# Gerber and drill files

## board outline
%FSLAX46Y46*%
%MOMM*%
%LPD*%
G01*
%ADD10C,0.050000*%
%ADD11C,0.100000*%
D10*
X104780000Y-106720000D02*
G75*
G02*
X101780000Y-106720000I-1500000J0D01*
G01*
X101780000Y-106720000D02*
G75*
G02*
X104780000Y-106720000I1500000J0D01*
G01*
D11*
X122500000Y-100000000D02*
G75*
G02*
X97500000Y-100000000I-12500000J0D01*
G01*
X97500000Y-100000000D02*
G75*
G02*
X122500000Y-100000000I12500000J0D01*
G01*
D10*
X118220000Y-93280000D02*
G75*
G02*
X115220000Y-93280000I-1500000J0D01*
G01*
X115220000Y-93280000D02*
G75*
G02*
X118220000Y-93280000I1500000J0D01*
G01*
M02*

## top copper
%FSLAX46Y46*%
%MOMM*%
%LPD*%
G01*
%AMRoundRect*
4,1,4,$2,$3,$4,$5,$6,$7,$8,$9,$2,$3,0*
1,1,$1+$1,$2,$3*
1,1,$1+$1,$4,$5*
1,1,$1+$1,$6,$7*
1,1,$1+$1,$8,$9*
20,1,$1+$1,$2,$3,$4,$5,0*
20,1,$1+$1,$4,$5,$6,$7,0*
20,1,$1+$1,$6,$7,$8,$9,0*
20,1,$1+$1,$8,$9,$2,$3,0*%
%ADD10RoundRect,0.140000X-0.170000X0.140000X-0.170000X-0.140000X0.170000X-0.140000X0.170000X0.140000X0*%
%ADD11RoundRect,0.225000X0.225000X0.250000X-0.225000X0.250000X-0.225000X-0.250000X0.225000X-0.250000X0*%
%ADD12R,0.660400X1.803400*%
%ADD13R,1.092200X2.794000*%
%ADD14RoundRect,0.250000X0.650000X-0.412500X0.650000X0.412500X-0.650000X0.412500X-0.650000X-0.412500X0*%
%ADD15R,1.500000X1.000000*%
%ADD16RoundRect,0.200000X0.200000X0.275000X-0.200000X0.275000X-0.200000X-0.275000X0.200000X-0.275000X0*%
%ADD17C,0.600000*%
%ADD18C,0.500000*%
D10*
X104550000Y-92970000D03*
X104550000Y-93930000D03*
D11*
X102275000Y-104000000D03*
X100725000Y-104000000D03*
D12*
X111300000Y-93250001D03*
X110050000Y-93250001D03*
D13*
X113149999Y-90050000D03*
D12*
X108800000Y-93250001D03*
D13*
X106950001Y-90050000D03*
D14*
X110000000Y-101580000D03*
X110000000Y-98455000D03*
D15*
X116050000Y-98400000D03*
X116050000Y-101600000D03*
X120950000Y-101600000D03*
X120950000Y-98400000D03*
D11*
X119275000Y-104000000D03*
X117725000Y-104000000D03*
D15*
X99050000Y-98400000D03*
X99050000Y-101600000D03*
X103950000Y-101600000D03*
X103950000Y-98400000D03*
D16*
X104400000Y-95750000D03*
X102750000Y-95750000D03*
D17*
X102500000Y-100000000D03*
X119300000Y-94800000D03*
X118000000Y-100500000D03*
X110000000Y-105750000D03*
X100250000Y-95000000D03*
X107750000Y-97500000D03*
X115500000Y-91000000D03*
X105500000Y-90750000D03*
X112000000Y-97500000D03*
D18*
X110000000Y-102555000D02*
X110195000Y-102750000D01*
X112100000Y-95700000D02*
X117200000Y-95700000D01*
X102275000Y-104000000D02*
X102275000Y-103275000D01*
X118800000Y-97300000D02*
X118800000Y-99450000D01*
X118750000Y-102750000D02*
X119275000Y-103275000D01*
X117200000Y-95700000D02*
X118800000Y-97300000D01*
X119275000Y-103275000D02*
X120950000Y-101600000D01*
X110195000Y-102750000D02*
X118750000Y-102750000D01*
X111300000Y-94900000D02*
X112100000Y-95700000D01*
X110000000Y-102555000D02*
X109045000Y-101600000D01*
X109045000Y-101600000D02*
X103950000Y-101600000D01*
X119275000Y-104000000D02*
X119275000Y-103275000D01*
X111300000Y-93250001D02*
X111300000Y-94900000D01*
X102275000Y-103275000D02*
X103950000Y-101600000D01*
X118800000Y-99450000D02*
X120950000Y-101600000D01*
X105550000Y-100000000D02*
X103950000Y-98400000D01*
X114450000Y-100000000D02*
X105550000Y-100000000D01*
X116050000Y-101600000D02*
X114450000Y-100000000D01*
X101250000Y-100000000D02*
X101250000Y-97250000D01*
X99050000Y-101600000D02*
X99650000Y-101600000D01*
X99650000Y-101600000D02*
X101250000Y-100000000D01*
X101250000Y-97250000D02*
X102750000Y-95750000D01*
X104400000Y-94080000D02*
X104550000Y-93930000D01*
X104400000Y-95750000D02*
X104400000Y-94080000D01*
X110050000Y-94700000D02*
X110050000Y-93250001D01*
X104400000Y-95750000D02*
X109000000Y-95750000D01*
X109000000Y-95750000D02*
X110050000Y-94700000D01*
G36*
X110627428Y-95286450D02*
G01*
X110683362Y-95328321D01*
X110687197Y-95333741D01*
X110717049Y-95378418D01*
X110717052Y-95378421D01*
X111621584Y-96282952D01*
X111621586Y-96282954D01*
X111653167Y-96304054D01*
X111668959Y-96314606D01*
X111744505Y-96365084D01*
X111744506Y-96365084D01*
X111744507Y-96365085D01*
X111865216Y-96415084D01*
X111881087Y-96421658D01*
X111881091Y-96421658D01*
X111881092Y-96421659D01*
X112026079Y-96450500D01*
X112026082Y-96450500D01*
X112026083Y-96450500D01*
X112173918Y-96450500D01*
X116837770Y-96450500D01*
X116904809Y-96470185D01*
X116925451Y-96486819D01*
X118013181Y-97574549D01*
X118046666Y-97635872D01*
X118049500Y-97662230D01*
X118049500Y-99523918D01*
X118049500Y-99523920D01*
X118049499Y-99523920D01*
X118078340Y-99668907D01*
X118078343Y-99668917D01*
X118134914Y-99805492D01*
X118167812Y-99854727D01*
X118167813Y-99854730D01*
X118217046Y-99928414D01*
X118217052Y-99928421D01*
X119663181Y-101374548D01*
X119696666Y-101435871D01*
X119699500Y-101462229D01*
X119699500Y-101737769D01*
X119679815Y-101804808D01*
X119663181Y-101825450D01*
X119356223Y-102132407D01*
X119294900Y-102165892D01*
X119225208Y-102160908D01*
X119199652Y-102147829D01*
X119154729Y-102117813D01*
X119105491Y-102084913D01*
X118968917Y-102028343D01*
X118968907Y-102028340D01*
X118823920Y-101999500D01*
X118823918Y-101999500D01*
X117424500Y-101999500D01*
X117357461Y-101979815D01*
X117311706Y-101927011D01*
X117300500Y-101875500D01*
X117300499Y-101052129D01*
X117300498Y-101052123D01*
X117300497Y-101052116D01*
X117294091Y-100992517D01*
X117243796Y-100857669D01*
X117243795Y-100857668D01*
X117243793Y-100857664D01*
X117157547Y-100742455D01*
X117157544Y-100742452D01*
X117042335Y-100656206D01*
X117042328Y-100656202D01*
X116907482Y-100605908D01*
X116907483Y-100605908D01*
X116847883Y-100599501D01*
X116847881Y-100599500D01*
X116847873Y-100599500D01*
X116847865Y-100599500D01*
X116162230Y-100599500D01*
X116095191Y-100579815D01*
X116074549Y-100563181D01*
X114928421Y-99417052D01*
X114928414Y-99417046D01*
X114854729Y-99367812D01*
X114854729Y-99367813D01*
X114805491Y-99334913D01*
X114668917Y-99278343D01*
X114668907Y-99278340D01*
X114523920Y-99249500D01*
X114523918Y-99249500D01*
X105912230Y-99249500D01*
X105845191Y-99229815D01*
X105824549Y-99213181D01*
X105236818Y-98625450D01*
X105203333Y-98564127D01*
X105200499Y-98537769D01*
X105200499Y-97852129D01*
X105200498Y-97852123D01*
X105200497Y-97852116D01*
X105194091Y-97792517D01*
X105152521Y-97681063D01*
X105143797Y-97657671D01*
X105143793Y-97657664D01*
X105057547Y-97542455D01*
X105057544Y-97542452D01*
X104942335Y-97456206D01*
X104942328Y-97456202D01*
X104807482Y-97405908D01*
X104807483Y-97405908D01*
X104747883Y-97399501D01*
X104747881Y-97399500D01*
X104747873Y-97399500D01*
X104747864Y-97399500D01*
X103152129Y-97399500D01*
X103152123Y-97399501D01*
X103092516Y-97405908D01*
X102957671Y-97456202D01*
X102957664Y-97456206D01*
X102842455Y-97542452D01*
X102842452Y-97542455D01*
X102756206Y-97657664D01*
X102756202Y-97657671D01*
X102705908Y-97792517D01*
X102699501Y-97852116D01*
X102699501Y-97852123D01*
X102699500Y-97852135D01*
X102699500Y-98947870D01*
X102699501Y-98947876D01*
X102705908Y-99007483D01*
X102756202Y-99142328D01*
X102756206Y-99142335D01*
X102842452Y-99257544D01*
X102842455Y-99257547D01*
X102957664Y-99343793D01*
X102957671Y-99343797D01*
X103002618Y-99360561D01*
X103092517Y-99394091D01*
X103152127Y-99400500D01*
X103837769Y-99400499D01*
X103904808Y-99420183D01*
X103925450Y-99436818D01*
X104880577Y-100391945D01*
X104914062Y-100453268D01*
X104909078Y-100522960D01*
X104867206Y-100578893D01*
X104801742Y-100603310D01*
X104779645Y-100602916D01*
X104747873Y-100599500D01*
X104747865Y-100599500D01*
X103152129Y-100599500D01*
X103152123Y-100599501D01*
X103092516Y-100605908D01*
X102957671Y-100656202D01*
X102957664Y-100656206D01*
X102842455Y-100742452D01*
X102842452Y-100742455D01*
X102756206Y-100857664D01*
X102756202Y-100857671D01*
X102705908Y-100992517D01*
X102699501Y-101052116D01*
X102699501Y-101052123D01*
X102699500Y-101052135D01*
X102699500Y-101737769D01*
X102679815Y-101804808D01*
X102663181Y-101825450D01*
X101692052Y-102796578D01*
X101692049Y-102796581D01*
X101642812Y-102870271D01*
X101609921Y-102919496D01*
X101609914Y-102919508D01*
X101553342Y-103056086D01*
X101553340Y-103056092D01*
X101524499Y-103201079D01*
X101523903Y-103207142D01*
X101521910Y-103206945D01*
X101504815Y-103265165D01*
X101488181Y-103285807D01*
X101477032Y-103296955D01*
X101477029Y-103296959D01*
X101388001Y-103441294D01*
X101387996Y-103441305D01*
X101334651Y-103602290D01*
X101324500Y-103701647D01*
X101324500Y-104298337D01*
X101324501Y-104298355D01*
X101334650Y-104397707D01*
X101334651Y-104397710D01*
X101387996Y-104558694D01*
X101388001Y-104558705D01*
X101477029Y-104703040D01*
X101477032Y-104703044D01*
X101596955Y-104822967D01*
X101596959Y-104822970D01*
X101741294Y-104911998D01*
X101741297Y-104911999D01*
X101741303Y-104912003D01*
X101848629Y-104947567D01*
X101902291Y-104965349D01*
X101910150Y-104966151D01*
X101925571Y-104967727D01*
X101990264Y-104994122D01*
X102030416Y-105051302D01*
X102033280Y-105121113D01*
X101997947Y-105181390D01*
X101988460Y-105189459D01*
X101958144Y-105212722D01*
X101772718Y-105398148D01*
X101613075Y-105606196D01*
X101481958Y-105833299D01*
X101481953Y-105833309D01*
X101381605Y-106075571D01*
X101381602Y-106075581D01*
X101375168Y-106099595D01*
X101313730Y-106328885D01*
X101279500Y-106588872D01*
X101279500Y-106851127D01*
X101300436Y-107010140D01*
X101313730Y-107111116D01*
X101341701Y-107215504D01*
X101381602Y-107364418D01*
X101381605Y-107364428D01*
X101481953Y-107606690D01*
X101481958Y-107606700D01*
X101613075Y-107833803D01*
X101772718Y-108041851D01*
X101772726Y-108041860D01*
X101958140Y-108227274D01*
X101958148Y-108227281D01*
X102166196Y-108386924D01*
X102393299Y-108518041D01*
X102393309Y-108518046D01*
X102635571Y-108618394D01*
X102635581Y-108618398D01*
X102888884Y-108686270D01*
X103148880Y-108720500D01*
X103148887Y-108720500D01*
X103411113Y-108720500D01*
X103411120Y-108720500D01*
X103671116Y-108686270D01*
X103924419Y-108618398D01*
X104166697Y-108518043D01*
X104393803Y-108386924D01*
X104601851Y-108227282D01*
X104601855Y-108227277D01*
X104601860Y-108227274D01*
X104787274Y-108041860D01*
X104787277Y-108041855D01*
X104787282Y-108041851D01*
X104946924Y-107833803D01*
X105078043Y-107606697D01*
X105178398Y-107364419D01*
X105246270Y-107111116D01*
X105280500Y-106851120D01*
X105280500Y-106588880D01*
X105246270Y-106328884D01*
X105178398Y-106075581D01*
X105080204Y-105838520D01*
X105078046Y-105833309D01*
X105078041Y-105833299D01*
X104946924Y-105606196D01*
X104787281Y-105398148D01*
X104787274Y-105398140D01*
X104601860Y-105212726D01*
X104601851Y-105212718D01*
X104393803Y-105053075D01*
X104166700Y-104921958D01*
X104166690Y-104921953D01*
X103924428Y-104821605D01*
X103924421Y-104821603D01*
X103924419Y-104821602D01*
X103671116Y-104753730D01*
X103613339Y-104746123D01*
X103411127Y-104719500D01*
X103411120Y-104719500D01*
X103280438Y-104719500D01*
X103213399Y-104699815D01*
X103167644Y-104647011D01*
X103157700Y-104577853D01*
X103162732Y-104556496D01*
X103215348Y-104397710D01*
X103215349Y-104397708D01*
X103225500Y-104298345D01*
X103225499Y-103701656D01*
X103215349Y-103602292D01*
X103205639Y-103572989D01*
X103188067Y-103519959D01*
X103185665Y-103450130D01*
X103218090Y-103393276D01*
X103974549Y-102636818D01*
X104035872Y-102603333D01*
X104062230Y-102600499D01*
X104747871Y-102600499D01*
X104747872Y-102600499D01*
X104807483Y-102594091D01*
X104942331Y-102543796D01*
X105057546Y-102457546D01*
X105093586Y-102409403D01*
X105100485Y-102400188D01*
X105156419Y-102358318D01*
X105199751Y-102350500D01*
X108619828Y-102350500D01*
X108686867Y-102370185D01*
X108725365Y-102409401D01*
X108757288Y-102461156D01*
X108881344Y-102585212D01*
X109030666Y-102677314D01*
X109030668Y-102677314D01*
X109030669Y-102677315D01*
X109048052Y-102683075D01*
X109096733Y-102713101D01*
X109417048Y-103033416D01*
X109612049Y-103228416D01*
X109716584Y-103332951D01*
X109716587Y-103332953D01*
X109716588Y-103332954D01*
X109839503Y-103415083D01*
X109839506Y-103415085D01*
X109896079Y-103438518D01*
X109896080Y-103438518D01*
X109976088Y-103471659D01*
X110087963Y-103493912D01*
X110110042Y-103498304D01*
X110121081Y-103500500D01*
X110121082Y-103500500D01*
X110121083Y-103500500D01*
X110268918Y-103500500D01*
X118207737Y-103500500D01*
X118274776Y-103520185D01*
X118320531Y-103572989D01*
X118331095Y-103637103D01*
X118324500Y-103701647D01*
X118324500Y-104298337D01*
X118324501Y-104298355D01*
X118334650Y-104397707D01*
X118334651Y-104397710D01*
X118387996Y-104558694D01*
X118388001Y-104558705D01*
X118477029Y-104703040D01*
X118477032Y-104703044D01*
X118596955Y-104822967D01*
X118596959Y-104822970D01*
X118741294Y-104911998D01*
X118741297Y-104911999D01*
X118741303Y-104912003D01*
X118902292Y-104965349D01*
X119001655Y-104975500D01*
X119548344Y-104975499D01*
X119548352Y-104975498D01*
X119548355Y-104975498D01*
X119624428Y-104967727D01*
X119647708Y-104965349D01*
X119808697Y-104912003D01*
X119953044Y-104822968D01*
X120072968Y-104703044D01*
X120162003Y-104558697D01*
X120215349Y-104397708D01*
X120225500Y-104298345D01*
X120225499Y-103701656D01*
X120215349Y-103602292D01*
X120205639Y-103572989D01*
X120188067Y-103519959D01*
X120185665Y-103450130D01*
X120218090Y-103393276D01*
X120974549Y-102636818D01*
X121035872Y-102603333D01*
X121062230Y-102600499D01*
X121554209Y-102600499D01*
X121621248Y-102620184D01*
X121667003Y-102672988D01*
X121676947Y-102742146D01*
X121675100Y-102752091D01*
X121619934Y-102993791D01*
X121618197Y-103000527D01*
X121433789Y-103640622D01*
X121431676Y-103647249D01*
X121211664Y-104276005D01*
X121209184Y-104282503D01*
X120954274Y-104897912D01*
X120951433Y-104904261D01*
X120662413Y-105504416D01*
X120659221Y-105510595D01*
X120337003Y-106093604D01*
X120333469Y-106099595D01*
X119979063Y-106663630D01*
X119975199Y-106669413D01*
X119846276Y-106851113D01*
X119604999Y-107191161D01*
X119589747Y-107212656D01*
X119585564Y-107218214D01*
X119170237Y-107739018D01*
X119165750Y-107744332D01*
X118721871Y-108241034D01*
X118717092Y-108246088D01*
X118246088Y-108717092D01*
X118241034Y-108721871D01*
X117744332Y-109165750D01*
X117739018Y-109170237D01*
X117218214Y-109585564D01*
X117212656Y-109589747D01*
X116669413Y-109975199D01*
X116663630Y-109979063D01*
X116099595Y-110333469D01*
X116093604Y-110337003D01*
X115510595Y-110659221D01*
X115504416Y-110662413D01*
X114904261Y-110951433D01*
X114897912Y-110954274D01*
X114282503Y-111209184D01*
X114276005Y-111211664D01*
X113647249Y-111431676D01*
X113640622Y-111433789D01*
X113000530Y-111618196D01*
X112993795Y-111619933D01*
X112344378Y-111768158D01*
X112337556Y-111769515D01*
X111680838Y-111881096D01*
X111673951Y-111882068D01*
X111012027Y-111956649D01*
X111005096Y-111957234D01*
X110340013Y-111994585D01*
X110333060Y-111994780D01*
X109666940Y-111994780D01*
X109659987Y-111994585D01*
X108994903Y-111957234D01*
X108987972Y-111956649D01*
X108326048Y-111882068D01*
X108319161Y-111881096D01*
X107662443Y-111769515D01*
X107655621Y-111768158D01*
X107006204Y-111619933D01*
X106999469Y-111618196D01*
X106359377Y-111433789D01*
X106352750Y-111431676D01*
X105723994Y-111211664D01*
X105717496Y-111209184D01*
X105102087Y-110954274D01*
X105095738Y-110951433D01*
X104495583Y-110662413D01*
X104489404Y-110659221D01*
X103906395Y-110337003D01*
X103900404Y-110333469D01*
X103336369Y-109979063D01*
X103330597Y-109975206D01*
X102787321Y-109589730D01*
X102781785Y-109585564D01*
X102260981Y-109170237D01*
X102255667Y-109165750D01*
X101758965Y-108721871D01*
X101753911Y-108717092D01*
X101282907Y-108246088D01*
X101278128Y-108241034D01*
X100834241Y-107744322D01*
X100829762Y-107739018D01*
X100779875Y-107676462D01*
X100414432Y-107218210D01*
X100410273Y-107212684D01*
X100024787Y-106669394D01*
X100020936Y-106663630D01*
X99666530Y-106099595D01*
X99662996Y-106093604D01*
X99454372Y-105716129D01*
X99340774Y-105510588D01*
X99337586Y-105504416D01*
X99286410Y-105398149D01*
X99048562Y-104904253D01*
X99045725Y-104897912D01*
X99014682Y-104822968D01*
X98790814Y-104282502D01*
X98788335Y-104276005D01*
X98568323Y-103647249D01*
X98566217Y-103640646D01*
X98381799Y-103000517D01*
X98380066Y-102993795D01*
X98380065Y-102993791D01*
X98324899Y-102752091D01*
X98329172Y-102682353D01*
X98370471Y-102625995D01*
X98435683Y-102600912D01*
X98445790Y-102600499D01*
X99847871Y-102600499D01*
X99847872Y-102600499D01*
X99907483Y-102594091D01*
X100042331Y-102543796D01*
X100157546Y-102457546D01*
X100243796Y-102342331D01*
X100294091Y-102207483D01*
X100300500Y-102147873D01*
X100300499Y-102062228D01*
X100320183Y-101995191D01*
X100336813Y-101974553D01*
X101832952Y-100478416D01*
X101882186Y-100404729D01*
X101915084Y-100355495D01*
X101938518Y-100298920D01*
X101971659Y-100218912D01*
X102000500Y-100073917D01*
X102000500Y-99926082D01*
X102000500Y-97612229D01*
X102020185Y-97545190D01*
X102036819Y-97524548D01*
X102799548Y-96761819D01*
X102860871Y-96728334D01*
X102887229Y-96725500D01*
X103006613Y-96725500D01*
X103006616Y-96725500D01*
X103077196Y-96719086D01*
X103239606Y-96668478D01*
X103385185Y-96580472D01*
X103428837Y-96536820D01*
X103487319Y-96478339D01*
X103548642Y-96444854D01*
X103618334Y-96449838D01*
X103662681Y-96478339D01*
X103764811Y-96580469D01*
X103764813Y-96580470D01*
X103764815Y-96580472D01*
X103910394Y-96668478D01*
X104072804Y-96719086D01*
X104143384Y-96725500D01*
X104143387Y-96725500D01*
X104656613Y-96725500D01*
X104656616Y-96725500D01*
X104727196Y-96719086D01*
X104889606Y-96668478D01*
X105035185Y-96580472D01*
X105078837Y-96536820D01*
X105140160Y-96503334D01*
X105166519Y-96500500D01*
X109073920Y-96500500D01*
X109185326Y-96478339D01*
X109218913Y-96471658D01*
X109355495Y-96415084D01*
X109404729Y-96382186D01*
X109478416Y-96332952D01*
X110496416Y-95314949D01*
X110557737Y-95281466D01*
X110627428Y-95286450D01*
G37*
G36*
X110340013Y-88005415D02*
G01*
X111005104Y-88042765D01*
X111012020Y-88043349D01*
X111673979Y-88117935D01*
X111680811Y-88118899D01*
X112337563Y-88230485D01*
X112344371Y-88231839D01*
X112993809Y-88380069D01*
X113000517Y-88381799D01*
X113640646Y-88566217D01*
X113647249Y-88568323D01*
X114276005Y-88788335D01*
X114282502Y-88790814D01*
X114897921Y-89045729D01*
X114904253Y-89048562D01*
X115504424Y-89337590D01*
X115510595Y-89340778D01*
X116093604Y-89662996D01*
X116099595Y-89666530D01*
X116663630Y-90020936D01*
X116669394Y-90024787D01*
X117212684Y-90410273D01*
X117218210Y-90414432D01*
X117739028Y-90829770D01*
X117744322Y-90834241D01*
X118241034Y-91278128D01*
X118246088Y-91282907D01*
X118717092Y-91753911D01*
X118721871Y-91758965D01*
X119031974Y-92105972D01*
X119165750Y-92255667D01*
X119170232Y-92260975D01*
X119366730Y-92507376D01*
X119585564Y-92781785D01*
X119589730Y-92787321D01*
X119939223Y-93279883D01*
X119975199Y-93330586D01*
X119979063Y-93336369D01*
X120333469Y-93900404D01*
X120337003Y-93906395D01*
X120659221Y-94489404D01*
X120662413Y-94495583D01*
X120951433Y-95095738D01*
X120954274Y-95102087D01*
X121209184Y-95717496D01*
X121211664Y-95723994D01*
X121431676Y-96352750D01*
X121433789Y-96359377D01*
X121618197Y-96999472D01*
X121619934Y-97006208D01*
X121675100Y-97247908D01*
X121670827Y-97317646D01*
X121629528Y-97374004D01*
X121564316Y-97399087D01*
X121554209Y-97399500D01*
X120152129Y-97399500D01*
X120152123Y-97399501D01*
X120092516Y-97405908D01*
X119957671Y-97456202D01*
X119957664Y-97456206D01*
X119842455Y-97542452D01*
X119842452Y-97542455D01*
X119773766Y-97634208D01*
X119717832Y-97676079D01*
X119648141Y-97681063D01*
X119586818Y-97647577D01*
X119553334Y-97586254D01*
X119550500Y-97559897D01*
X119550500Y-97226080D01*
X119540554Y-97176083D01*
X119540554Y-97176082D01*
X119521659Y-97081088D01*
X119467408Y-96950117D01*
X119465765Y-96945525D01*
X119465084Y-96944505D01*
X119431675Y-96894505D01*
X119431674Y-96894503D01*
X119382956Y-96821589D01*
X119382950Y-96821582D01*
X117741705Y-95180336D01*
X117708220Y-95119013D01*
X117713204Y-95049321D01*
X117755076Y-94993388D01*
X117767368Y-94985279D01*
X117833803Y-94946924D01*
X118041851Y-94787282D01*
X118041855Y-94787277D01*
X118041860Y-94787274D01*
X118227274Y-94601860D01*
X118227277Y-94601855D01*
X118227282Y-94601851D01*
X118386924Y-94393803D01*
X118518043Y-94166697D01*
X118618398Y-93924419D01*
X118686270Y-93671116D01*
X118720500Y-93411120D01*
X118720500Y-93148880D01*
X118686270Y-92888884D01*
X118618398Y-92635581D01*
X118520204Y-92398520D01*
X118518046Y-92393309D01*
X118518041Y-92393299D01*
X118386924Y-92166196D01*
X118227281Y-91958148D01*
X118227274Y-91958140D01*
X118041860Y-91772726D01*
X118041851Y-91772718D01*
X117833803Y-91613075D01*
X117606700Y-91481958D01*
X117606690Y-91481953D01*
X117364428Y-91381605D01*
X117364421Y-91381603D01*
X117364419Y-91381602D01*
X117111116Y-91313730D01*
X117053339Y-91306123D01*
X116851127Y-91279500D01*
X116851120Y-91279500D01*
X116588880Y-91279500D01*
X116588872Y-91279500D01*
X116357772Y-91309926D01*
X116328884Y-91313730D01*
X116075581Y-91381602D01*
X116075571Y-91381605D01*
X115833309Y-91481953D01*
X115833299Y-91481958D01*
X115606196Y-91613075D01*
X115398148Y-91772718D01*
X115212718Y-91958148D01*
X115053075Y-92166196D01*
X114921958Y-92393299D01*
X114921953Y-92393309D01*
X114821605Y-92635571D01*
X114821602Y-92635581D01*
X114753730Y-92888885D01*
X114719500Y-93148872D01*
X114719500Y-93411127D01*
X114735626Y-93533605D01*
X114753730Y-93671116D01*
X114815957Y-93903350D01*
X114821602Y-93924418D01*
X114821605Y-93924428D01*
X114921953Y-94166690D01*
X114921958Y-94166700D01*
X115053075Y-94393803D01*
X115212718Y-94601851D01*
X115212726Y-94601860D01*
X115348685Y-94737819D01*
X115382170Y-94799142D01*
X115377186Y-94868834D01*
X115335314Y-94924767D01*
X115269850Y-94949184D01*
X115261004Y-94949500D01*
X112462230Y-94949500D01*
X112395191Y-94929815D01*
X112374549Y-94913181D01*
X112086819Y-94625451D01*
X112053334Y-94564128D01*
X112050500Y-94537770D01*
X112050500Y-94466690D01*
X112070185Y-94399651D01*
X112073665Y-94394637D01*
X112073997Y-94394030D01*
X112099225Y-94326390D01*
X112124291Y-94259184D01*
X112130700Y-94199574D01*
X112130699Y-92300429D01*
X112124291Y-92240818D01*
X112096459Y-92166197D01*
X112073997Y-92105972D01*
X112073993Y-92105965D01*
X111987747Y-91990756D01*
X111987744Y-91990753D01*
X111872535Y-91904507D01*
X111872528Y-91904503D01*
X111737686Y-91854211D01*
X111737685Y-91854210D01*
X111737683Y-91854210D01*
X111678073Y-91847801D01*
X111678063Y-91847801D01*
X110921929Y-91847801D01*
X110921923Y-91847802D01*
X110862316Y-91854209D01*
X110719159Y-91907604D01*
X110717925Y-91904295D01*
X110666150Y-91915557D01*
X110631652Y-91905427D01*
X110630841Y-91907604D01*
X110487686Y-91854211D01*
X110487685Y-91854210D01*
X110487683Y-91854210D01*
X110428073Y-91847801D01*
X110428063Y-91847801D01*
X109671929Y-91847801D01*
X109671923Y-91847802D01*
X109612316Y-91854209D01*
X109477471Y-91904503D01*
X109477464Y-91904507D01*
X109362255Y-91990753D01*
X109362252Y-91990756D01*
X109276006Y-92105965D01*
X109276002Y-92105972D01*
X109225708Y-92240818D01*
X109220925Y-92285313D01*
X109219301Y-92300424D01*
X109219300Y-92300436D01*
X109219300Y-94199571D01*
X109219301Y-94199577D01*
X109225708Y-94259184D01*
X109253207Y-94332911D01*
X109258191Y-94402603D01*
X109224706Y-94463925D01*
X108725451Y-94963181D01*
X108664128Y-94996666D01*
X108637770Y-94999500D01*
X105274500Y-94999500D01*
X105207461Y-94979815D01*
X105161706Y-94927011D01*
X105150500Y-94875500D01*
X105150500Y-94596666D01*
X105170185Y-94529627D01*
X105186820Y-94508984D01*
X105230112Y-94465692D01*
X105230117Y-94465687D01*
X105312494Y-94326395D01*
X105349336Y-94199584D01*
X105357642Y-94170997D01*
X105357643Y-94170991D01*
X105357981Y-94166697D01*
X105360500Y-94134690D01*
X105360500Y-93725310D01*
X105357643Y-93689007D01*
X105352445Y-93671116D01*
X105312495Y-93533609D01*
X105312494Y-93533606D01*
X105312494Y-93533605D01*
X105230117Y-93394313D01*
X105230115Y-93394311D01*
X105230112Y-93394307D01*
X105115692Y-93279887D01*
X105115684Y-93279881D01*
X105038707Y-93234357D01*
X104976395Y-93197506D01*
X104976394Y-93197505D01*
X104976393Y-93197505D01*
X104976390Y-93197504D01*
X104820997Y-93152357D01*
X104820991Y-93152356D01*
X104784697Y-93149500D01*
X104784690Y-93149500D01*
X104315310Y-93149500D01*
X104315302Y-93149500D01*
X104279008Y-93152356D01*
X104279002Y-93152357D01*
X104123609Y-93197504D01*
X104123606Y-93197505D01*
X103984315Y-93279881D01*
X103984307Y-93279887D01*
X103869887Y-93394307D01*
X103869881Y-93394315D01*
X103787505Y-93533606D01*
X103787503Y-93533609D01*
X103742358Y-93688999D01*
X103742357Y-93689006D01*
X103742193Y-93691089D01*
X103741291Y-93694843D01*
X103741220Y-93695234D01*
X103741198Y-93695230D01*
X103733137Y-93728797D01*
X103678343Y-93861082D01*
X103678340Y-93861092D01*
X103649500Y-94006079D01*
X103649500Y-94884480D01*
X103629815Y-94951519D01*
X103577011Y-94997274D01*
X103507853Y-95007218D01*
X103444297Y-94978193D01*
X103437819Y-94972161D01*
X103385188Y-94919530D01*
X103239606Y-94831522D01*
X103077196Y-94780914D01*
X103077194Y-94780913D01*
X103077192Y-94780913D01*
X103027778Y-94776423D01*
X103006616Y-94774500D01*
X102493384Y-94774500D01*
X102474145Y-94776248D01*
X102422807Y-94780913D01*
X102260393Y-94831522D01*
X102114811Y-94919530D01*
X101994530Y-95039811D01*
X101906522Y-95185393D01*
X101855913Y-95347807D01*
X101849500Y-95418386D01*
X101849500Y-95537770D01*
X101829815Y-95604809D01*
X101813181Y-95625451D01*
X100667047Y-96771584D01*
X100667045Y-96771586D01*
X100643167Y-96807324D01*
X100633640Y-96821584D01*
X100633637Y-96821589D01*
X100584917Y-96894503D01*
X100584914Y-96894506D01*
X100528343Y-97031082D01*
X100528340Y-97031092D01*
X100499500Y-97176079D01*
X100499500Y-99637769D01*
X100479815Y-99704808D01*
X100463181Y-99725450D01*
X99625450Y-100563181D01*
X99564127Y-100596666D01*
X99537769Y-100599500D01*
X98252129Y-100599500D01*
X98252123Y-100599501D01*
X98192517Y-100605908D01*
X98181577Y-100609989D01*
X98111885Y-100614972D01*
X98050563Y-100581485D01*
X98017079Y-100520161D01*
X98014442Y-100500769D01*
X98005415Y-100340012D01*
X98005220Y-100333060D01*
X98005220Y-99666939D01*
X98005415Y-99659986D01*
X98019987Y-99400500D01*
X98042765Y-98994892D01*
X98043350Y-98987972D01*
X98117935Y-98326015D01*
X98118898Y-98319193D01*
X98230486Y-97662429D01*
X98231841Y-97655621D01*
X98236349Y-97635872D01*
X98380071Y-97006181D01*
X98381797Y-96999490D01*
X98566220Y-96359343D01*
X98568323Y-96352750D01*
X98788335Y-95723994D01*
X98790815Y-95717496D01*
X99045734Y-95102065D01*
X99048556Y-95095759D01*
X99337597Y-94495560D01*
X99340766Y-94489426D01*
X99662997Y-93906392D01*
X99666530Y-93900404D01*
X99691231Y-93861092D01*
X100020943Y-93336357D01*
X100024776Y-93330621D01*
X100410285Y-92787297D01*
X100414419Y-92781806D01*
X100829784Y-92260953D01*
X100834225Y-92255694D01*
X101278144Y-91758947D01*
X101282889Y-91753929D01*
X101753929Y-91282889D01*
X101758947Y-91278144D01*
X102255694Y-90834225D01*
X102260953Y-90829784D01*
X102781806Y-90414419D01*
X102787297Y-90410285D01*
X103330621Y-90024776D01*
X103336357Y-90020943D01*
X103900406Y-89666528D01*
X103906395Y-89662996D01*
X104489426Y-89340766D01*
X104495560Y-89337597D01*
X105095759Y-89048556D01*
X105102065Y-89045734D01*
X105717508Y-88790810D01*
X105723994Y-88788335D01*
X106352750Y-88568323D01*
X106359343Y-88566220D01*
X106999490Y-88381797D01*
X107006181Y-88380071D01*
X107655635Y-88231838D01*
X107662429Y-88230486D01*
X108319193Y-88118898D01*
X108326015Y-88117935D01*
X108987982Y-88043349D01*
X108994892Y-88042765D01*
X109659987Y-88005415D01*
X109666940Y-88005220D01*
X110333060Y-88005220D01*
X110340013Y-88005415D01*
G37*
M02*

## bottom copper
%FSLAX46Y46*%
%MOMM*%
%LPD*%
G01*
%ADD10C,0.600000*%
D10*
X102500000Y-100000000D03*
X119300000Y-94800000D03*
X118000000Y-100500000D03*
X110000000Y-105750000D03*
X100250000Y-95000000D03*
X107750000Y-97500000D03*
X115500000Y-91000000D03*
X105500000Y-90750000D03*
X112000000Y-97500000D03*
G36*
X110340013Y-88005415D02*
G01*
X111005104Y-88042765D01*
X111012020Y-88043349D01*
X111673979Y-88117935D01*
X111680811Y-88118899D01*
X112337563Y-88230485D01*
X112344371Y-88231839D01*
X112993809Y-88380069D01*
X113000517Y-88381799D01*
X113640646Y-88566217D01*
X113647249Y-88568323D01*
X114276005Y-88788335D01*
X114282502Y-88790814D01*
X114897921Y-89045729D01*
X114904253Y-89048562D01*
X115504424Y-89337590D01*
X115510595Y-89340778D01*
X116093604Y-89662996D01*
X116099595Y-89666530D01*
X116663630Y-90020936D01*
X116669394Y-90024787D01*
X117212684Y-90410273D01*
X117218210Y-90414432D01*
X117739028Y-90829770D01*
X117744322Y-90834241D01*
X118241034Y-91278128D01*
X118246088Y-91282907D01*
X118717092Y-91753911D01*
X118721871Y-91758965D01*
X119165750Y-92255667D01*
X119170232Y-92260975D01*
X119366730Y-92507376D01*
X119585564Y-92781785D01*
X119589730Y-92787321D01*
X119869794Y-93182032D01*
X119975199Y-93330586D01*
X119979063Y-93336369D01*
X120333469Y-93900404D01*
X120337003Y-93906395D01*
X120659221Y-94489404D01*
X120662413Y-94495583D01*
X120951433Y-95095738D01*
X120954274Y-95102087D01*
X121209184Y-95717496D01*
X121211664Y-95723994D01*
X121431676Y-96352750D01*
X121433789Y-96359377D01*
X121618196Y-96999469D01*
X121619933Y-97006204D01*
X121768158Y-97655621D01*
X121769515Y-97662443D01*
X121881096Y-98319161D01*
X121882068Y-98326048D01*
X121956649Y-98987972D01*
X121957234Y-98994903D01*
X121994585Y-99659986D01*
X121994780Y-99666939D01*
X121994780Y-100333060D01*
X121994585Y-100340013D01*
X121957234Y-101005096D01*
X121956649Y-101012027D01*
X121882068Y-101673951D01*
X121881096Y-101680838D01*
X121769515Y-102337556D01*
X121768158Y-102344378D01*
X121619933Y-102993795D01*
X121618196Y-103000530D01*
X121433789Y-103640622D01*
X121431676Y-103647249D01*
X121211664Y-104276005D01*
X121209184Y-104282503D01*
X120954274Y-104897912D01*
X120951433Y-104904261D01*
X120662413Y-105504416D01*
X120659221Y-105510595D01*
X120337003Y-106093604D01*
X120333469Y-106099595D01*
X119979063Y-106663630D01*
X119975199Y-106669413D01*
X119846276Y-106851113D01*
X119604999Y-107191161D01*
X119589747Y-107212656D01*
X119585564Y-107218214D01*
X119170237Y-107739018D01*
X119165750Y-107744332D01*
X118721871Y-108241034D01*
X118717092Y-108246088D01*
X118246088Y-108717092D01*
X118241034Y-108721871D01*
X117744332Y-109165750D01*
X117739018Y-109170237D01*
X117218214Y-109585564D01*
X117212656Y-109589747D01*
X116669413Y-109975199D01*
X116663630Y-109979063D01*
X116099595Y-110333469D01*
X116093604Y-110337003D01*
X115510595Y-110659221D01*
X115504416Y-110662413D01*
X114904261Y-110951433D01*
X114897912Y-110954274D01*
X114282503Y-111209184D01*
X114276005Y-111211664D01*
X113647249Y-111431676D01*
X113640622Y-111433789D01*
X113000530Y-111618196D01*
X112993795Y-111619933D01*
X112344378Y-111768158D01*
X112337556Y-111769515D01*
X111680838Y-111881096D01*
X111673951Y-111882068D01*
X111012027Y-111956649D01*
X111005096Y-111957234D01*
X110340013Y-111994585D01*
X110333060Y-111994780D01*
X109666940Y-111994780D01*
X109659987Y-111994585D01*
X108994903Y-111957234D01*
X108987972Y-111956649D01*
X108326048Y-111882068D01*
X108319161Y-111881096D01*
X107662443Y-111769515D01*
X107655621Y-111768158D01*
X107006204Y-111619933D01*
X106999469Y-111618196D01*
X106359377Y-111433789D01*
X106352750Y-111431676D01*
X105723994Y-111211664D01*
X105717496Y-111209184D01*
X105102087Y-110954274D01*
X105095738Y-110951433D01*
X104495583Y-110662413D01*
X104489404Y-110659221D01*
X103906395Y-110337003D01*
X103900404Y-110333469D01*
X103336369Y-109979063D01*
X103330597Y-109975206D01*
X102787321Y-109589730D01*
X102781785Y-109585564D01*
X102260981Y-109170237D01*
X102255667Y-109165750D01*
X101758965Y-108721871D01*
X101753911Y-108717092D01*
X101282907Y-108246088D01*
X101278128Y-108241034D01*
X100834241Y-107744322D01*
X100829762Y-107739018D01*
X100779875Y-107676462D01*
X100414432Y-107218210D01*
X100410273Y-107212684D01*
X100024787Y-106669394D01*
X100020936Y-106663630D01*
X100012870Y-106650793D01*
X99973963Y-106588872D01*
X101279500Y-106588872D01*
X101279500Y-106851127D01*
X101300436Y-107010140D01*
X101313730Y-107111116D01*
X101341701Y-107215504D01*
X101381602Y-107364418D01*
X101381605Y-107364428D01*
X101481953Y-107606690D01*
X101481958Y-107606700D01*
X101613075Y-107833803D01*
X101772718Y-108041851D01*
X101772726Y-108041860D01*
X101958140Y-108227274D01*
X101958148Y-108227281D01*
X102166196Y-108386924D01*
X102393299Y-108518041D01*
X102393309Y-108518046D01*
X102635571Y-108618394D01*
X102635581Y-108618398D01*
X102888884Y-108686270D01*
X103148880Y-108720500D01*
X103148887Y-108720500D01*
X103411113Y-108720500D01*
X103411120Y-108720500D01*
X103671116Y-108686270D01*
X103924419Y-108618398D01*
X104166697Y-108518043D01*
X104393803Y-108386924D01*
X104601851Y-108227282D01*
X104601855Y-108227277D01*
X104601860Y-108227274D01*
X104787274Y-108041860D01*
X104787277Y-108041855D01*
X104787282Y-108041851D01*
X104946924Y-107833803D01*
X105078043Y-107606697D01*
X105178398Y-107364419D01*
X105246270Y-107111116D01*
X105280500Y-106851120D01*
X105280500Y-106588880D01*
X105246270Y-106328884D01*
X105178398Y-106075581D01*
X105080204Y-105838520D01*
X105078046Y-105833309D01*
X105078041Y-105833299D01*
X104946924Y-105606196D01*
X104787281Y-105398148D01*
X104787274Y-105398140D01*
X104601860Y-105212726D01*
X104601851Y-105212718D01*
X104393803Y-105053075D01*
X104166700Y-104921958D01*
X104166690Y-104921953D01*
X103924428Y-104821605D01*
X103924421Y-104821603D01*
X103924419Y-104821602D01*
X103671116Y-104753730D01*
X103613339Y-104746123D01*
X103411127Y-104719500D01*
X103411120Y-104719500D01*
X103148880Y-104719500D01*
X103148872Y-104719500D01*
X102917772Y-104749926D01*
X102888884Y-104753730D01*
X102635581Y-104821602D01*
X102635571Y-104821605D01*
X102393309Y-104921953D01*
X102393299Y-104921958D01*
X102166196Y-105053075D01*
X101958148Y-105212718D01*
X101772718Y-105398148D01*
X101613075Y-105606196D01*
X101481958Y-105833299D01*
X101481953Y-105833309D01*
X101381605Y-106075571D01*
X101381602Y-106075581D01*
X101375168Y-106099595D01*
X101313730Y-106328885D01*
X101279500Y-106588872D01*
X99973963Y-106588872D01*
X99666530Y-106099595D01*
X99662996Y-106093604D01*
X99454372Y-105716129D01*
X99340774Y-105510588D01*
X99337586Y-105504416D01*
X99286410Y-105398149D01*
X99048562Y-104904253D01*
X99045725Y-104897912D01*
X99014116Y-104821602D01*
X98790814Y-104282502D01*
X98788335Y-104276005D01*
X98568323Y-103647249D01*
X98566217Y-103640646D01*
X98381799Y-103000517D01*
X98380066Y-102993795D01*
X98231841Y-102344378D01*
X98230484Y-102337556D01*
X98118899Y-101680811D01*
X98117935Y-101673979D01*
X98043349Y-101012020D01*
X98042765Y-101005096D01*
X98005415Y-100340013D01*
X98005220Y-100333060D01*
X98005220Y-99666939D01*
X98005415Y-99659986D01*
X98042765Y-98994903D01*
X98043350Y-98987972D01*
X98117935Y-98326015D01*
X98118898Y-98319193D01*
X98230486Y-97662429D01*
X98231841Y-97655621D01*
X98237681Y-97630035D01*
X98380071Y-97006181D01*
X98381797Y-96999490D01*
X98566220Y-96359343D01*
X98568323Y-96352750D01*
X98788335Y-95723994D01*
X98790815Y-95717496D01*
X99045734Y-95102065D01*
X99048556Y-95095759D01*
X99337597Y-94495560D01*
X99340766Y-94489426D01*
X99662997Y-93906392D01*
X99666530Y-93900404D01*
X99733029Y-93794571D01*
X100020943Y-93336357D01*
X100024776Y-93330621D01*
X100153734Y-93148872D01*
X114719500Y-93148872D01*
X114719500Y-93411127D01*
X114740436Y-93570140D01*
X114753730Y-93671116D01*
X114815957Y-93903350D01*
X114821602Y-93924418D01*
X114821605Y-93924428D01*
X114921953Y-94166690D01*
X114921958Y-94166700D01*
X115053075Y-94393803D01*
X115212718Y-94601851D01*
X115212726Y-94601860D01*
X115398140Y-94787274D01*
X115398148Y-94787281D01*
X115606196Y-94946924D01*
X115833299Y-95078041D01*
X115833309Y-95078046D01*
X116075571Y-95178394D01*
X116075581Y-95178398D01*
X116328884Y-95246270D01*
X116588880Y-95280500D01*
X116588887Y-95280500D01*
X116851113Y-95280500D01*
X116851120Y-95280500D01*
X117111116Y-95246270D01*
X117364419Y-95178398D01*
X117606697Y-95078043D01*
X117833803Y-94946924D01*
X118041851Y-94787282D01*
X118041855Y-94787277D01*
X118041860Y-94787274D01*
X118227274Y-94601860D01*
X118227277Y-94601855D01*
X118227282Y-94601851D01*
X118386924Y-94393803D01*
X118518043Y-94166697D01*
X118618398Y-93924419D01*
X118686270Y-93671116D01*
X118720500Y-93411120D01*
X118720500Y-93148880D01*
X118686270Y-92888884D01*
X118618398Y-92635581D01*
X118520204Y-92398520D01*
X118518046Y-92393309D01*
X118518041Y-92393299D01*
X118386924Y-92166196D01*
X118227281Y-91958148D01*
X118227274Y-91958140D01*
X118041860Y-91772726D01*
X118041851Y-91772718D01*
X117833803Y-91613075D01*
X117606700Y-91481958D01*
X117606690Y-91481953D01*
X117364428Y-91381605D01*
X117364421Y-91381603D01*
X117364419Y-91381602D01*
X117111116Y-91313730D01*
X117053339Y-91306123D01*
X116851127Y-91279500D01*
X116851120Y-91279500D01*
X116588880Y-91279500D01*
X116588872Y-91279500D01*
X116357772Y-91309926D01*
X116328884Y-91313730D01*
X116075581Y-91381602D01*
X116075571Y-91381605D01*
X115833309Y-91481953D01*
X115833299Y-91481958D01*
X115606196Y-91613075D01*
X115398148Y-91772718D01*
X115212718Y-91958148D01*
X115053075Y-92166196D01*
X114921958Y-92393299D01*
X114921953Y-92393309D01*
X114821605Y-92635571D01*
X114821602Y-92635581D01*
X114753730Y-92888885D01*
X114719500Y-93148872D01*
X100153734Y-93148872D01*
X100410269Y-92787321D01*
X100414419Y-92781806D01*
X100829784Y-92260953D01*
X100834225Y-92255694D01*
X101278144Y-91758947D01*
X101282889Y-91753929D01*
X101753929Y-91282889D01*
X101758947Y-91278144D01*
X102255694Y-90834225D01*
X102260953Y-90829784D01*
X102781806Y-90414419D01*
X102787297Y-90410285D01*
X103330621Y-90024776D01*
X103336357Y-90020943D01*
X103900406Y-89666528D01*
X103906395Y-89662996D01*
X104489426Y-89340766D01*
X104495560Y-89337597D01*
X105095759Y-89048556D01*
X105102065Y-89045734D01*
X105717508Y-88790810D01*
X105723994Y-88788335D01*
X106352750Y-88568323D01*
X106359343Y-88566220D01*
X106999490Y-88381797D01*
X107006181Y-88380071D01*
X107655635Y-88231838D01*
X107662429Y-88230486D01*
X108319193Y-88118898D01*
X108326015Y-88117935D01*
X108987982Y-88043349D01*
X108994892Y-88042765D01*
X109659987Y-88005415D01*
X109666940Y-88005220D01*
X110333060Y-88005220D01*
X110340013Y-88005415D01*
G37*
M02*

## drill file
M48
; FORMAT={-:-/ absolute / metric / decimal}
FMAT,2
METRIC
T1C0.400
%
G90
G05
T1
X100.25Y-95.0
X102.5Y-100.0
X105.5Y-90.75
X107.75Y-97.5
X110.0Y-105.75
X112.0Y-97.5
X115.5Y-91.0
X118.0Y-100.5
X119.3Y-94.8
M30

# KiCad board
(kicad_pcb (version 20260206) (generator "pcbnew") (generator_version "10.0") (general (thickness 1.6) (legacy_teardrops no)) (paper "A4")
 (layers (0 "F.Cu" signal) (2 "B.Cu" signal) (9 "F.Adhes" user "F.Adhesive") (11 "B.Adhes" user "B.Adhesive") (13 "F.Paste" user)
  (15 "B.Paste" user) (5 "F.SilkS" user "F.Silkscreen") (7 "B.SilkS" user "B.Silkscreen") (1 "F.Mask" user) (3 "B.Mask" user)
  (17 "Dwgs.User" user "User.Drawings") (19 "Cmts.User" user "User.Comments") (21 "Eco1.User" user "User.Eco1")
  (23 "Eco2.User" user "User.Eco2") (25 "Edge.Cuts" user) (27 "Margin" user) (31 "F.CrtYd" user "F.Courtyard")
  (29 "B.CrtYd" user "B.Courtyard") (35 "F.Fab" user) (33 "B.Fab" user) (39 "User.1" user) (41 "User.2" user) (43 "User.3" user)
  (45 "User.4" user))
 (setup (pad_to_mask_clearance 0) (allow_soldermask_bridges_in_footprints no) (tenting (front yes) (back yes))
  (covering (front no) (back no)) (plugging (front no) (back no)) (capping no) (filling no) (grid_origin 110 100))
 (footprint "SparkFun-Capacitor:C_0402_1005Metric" (layer "F.Cu") (at 104.55 93.45 -90)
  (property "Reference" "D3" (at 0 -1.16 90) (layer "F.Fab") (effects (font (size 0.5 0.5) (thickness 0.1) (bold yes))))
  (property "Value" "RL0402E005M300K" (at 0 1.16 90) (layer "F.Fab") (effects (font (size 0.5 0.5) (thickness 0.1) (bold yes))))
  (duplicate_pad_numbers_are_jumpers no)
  (pad "1" smd roundrect (at -0.48 0 270) (size 0.56 0.62) (layers "F.Cu" "F.Mask" "F.Paste") (roundrect_rratio 0.25) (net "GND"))
  (pad "2" smd roundrect (at 0.48 0 270) (size 0.56 0.62) (layers "F.Cu" "F.Mask" "F.Paste") (roundrect_rratio 0.25) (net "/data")))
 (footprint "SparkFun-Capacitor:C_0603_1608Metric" (layer "F.Cu") (at 101.5 104 180)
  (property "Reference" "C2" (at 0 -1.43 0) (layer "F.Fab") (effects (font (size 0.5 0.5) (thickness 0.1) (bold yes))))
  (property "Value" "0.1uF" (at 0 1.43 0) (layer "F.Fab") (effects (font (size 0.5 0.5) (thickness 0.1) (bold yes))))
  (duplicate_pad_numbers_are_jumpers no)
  (pad "1" smd roundrect (at -0.775 0 180) (size 0.9 0.95) (layers "F.Cu" "F.Mask" "F.Paste") (roundrect_rratio 0.25) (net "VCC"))
  (pad "2" smd roundrect (at 0.775 0 180) (size 0.9 0.95) (layers "F.Cu" "F.Mask" "F.Paste") (roundrect_rratio 0.25) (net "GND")))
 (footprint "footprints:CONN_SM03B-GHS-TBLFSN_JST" (layer "F.Cu") (at 110.05 91.046297 180)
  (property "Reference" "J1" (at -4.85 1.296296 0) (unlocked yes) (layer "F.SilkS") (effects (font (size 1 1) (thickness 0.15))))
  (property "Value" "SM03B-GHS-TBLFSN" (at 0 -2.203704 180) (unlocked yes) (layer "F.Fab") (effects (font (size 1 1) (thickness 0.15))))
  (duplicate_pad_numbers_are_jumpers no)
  (pad "1" smd rect (at -1.25 -2.203704 180) (size 0.6604 1.8034) (layers "F.Cu" "F.Mask" "F.Paste") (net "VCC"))
  (pad "2" smd rect (at 0 -2.203704 180) (size 0.6604 1.8034) (layers "F.Cu" "F.Mask" "F.Paste") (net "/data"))
  (pad "3" smd rect (at -3.099999 0.996297 180) (size 1.0922 2.794) (layers "F.Cu" "F.Mask" "F.Paste") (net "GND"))
  (pad "3" smd rect (at 1.25 -2.203704 180) (size 0.6604 1.8034) (layers "F.Cu" "F.Mask" "F.Paste") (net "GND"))
  (pad "3" smd rect (at 3.099999 0.996297 180) (size 1.0922 2.794) (layers "F.Cu" "F.Mask" "F.Paste") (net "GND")))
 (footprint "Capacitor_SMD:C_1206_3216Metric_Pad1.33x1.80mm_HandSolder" (layer "F.Cu") (at 110 100.0175 90)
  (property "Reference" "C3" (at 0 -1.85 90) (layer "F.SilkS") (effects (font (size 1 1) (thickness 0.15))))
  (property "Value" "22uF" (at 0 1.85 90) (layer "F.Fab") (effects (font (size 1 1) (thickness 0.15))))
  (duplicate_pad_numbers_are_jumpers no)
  (pad "1" smd roundrect (at -1.5625 0 90) (size 1.325 1.8) (layers "F.Cu" "F.Mask" "F.Paste") (roundrect_rratio 0.188679) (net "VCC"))
  (pad "2" smd roundrect (at 1.5625 0 90) (size 1.325 1.8) (layers "F.Cu" "F.Mask" "F.Paste") (roundrect_rratio 0.188679) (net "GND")))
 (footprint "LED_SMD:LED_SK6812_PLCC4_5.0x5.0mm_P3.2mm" (layer "F.Cu") (at 118.5 100)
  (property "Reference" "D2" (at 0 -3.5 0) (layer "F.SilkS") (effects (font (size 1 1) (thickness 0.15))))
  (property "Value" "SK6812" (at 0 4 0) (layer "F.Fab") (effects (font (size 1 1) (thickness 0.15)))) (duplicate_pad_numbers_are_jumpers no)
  (pad "1" smd rect (at -2.45 -1.6 180) (size 1.5 1) (layers "F.Cu" "F.Mask" "F.Paste") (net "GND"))
  (pad "2" smd rect (at -2.45 1.6 180) (size 1.5 1) (layers "F.Cu" "F.Mask" "F.Paste") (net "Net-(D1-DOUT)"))
  (pad "3" smd rect (at 2.45 1.6 180) (size 1.5 1) (layers "F.Cu" "F.Mask" "F.Paste") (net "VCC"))
  (pad "4" smd rect (at 2.45 -1.6 180) (size 1.5 1) (layers "F.Cu" "F.Mask" "F.Paste") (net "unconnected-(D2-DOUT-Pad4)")))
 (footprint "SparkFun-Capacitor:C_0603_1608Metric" (layer "F.Cu") (at 118.5 104 180)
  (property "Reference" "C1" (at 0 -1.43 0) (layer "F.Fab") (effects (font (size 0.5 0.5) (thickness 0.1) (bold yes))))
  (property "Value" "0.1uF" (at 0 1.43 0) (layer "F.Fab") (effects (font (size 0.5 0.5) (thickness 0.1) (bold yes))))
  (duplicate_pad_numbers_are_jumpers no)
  (pad "1" smd roundrect (at -0.775 0 180) (size 0.9 0.95) (layers "F.Cu" "F.Mask" "F.Paste") (roundrect_rratio 0.25) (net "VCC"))
  (pad "2" smd roundrect (at 0.775 0 180) (size 0.9 0.95) (layers "F.Cu" "F.Mask" "F.Paste") (roundrect_rratio 0.25) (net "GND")))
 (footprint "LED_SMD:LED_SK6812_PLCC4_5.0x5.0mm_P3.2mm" (layer "F.Cu") (at 101.5 100)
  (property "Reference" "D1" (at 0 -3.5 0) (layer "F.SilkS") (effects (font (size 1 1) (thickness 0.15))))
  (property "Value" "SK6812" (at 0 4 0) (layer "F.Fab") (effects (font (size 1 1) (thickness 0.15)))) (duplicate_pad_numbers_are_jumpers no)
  (pad "1" smd rect (at -2.45 -1.6 180) (size 1.5 1) (layers "F.Cu" "F.Mask" "F.Paste") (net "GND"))
  (pad "2" smd rect (at -2.45 1.6 180) (size 1.5 1) (layers "F.Cu" "F.Mask" "F.Paste") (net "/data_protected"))
  (pad "3" smd rect (at 2.45 1.6 180) (size 1.5 1) (layers "F.Cu" "F.Mask" "F.Paste") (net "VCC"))
  (pad "4" smd rect (at 2.45 -1.6 180) (size 1.5 1) (layers "F.Cu" "F.Mask" "F.Paste") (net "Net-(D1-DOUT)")))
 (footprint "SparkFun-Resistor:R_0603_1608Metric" (layer "F.Cu") (at 103.575 95.75 180)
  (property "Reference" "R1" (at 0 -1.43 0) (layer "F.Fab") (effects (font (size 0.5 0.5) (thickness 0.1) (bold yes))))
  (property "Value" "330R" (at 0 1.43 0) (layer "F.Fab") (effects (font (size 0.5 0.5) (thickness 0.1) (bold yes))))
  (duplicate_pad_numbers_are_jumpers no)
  (pad "1" smd roundrect (at -0.825 0 180) (size 0.8 0.95) (layers "F.Cu" "F.Mask" "F.Paste") (roundrect_rratio 0.25) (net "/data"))
  (pad "2" smd roundrect (at 0.825 0 180) (size 0.8 0.95) (layers "F.Cu" "F.Mask" "F.Paste") (roundrect_rratio 0.25) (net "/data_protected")))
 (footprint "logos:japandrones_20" (layer "B.Cu") (at 110 99 180)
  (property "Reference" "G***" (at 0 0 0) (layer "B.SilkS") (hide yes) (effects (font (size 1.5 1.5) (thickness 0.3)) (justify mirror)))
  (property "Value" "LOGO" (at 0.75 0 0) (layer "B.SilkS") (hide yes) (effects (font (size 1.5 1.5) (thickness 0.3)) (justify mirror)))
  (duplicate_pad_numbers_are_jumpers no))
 (gr_circle (center 103.28 106.72) (end 104.78 106.72) (stroke (width 0.05) (type solid)) (fill no) (layer "Edge.Cuts"))
 (gr_circle (center 110 100) (end 122.5 100) (stroke (width 0.1) (type solid)) (fill no) (layer "Edge.Cuts"))
 (gr_circle (center 116.72 93.28) (end 118.22 93.28) (stroke (width 0.05) (type solid)) (fill no) (layer "Edge.Cuts"))
 (via (at 102.5 100) (size 0.6) (drill 0.4) (layers "F.Cu" "B.Cu") (free yes) (capping no) (covering (front no) (back no))
  (plugging (front no) (back no)) (filling no) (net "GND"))
 (via (at 119.3 94.8) (size 0.6) (drill 0.4) (layers "F.Cu" "B.Cu") (free yes) (capping no) (covering (front no) (back no))
  (plugging (front no) (back no)) (filling no) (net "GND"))
 (via (at 118 100.5) (size 0.6) (drill 0.4) (layers "F.Cu" "B.Cu") (free yes) (capping no) (covering (front no) (back no))
  (plugging (front no) (back no)) (filling no) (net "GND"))
 (via (at 110 105.75) (size 0.6) (drill 0.4) (layers "F.Cu" "B.Cu") (free yes) (capping no) (covering (front no) (back no))
  (plugging (front no) (back no)) (filling no) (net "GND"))
 (via (at 100.25 95) (size 0.6) (drill 0.4) (layers "F.Cu" "B.Cu") (free yes) (capping no) (covering (front no) (back no))
  (plugging (front no) (back no)) (filling no) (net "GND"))
 (via (at 107.75 97.5) (size 0.6) (drill 0.4) (layers "F.Cu" "B.Cu") (free yes) (capping no) (covering (front no) (back no))
  (plugging (front no) (back no)) (filling no) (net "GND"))
 (via (at 115.5 91) (size 0.6) (drill 0.4) (layers "F.Cu" "B.Cu") (free yes) (capping no) (covering (front no) (back no))
  (plugging (front no) (back no)) (filling no) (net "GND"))
 (via (at 105.5 90.75) (size 0.6) (drill 0.4) (layers "F.Cu" "B.Cu") (free yes) (capping no) (covering (front no) (back no))
  (plugging (front no) (back no)) (filling no) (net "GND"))
 (via (at 112 97.5) (size 0.6) (drill 0.4) (layers "F.Cu" "B.Cu") (free yes) (capping no) (covering (front no) (back no))
  (plugging (front no) (back no)) (filling no) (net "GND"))
 (segment (start 110 102.555) (end 110.195 102.75) (width 0.5) (layer "F.Cu") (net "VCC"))
 (segment (start 112.1 95.7) (end 117.2 95.7) (width 0.5) (layer "F.Cu") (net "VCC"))
 (segment (start 102.275 104) (end 102.275 103.275) (width 0.5) (layer "F.Cu") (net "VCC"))
 (segment (start 118.8 97.3) (end 118.8 99.45) (width 0.5) (layer "F.Cu") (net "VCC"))
 (segment (start 118.75 102.75) (end 119.275 103.275) (width 0.5) (layer "F.Cu") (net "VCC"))
 (segment (start 117.2 95.7) (end 118.8 97.3) (width 0.5) (layer "F.Cu") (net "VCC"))
 (segment (start 119.275 103.275) (end 120.95 101.6) (width 0.5) (layer "F.Cu") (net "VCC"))
 (segment (start 110.195 102.75) (end 118.75 102.75) (width 0.5) (layer "F.Cu") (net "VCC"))
 (segment (start 111.3 94.9) (end 112.1 95.7) (width 0.5) (layer "F.Cu") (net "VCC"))
 (segment (start 110 102.555) (end 109.045 101.6) (width 0.5) (layer "F.Cu") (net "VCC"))
 (segment (start 109.045 101.6) (end 103.95 101.6) (width 0.5) (layer "F.Cu") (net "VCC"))
 (segment (start 119.275 104) (end 119.275 103.275) (width 0.5) (layer "F.Cu") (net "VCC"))
 (segment (start 111.3 93.250001) (end 111.3 94.9) (width 0.5) (layer "F.Cu") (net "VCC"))
 (segment (start 102.275 103.275) (end 103.95 101.6) (width 0.5) (layer "F.Cu") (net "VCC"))
 (segment (start 118.8 99.45) (end 120.95 101.6) (width 0.5) (layer "F.Cu") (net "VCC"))
 (segment (start 105.55 100) (end 103.95 98.4) (width 0.5) (layer "F.Cu") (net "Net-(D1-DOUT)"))
 (segment (start 114.45 100) (end 105.55 100) (width 0.5) (layer "F.Cu") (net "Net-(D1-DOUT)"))
 (segment (start 116.05 101.6) (end 114.45 100) (width 0.5) (layer "F.Cu") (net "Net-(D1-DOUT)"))
 (segment (start 101.25 100) (end 101.25 97.25) (width 0.5) (layer "F.Cu") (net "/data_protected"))
 (segment (start 99.05 101.6) (end 99.65 101.6) (width 0.5) (layer "F.Cu") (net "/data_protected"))
 (segment (start 99.65 101.6) (end 101.25 100) (width 0.5) (layer "F.Cu") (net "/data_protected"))
 (segment (start 101.25 97.25) (end 102.75 95.75) (width 0.5) (layer "F.Cu") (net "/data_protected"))
 (segment (start 104.4 94.08) (end 104.55 93.93) (width 0.5) (layer "F.Cu") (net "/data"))
 (segment (start 104.4 95.75) (end 104.4 94.08) (width 0.5) (layer "F.Cu") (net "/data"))
 (segment (start 110.05 94.7) (end 110.05 93.250001) (width 0.5) (layer "F.Cu") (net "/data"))
 (segment (start 104.4 95.75) (end 109 95.75) (width 0.5) (layer "F.Cu") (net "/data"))
 (segment (start 109 95.75) (end 110.05 94.7) (width 0.5) (layer "F.Cu") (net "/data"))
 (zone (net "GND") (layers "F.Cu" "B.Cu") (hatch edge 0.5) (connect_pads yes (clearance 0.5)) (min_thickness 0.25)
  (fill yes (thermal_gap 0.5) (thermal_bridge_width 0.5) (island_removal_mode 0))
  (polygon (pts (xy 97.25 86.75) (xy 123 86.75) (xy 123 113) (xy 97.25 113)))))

